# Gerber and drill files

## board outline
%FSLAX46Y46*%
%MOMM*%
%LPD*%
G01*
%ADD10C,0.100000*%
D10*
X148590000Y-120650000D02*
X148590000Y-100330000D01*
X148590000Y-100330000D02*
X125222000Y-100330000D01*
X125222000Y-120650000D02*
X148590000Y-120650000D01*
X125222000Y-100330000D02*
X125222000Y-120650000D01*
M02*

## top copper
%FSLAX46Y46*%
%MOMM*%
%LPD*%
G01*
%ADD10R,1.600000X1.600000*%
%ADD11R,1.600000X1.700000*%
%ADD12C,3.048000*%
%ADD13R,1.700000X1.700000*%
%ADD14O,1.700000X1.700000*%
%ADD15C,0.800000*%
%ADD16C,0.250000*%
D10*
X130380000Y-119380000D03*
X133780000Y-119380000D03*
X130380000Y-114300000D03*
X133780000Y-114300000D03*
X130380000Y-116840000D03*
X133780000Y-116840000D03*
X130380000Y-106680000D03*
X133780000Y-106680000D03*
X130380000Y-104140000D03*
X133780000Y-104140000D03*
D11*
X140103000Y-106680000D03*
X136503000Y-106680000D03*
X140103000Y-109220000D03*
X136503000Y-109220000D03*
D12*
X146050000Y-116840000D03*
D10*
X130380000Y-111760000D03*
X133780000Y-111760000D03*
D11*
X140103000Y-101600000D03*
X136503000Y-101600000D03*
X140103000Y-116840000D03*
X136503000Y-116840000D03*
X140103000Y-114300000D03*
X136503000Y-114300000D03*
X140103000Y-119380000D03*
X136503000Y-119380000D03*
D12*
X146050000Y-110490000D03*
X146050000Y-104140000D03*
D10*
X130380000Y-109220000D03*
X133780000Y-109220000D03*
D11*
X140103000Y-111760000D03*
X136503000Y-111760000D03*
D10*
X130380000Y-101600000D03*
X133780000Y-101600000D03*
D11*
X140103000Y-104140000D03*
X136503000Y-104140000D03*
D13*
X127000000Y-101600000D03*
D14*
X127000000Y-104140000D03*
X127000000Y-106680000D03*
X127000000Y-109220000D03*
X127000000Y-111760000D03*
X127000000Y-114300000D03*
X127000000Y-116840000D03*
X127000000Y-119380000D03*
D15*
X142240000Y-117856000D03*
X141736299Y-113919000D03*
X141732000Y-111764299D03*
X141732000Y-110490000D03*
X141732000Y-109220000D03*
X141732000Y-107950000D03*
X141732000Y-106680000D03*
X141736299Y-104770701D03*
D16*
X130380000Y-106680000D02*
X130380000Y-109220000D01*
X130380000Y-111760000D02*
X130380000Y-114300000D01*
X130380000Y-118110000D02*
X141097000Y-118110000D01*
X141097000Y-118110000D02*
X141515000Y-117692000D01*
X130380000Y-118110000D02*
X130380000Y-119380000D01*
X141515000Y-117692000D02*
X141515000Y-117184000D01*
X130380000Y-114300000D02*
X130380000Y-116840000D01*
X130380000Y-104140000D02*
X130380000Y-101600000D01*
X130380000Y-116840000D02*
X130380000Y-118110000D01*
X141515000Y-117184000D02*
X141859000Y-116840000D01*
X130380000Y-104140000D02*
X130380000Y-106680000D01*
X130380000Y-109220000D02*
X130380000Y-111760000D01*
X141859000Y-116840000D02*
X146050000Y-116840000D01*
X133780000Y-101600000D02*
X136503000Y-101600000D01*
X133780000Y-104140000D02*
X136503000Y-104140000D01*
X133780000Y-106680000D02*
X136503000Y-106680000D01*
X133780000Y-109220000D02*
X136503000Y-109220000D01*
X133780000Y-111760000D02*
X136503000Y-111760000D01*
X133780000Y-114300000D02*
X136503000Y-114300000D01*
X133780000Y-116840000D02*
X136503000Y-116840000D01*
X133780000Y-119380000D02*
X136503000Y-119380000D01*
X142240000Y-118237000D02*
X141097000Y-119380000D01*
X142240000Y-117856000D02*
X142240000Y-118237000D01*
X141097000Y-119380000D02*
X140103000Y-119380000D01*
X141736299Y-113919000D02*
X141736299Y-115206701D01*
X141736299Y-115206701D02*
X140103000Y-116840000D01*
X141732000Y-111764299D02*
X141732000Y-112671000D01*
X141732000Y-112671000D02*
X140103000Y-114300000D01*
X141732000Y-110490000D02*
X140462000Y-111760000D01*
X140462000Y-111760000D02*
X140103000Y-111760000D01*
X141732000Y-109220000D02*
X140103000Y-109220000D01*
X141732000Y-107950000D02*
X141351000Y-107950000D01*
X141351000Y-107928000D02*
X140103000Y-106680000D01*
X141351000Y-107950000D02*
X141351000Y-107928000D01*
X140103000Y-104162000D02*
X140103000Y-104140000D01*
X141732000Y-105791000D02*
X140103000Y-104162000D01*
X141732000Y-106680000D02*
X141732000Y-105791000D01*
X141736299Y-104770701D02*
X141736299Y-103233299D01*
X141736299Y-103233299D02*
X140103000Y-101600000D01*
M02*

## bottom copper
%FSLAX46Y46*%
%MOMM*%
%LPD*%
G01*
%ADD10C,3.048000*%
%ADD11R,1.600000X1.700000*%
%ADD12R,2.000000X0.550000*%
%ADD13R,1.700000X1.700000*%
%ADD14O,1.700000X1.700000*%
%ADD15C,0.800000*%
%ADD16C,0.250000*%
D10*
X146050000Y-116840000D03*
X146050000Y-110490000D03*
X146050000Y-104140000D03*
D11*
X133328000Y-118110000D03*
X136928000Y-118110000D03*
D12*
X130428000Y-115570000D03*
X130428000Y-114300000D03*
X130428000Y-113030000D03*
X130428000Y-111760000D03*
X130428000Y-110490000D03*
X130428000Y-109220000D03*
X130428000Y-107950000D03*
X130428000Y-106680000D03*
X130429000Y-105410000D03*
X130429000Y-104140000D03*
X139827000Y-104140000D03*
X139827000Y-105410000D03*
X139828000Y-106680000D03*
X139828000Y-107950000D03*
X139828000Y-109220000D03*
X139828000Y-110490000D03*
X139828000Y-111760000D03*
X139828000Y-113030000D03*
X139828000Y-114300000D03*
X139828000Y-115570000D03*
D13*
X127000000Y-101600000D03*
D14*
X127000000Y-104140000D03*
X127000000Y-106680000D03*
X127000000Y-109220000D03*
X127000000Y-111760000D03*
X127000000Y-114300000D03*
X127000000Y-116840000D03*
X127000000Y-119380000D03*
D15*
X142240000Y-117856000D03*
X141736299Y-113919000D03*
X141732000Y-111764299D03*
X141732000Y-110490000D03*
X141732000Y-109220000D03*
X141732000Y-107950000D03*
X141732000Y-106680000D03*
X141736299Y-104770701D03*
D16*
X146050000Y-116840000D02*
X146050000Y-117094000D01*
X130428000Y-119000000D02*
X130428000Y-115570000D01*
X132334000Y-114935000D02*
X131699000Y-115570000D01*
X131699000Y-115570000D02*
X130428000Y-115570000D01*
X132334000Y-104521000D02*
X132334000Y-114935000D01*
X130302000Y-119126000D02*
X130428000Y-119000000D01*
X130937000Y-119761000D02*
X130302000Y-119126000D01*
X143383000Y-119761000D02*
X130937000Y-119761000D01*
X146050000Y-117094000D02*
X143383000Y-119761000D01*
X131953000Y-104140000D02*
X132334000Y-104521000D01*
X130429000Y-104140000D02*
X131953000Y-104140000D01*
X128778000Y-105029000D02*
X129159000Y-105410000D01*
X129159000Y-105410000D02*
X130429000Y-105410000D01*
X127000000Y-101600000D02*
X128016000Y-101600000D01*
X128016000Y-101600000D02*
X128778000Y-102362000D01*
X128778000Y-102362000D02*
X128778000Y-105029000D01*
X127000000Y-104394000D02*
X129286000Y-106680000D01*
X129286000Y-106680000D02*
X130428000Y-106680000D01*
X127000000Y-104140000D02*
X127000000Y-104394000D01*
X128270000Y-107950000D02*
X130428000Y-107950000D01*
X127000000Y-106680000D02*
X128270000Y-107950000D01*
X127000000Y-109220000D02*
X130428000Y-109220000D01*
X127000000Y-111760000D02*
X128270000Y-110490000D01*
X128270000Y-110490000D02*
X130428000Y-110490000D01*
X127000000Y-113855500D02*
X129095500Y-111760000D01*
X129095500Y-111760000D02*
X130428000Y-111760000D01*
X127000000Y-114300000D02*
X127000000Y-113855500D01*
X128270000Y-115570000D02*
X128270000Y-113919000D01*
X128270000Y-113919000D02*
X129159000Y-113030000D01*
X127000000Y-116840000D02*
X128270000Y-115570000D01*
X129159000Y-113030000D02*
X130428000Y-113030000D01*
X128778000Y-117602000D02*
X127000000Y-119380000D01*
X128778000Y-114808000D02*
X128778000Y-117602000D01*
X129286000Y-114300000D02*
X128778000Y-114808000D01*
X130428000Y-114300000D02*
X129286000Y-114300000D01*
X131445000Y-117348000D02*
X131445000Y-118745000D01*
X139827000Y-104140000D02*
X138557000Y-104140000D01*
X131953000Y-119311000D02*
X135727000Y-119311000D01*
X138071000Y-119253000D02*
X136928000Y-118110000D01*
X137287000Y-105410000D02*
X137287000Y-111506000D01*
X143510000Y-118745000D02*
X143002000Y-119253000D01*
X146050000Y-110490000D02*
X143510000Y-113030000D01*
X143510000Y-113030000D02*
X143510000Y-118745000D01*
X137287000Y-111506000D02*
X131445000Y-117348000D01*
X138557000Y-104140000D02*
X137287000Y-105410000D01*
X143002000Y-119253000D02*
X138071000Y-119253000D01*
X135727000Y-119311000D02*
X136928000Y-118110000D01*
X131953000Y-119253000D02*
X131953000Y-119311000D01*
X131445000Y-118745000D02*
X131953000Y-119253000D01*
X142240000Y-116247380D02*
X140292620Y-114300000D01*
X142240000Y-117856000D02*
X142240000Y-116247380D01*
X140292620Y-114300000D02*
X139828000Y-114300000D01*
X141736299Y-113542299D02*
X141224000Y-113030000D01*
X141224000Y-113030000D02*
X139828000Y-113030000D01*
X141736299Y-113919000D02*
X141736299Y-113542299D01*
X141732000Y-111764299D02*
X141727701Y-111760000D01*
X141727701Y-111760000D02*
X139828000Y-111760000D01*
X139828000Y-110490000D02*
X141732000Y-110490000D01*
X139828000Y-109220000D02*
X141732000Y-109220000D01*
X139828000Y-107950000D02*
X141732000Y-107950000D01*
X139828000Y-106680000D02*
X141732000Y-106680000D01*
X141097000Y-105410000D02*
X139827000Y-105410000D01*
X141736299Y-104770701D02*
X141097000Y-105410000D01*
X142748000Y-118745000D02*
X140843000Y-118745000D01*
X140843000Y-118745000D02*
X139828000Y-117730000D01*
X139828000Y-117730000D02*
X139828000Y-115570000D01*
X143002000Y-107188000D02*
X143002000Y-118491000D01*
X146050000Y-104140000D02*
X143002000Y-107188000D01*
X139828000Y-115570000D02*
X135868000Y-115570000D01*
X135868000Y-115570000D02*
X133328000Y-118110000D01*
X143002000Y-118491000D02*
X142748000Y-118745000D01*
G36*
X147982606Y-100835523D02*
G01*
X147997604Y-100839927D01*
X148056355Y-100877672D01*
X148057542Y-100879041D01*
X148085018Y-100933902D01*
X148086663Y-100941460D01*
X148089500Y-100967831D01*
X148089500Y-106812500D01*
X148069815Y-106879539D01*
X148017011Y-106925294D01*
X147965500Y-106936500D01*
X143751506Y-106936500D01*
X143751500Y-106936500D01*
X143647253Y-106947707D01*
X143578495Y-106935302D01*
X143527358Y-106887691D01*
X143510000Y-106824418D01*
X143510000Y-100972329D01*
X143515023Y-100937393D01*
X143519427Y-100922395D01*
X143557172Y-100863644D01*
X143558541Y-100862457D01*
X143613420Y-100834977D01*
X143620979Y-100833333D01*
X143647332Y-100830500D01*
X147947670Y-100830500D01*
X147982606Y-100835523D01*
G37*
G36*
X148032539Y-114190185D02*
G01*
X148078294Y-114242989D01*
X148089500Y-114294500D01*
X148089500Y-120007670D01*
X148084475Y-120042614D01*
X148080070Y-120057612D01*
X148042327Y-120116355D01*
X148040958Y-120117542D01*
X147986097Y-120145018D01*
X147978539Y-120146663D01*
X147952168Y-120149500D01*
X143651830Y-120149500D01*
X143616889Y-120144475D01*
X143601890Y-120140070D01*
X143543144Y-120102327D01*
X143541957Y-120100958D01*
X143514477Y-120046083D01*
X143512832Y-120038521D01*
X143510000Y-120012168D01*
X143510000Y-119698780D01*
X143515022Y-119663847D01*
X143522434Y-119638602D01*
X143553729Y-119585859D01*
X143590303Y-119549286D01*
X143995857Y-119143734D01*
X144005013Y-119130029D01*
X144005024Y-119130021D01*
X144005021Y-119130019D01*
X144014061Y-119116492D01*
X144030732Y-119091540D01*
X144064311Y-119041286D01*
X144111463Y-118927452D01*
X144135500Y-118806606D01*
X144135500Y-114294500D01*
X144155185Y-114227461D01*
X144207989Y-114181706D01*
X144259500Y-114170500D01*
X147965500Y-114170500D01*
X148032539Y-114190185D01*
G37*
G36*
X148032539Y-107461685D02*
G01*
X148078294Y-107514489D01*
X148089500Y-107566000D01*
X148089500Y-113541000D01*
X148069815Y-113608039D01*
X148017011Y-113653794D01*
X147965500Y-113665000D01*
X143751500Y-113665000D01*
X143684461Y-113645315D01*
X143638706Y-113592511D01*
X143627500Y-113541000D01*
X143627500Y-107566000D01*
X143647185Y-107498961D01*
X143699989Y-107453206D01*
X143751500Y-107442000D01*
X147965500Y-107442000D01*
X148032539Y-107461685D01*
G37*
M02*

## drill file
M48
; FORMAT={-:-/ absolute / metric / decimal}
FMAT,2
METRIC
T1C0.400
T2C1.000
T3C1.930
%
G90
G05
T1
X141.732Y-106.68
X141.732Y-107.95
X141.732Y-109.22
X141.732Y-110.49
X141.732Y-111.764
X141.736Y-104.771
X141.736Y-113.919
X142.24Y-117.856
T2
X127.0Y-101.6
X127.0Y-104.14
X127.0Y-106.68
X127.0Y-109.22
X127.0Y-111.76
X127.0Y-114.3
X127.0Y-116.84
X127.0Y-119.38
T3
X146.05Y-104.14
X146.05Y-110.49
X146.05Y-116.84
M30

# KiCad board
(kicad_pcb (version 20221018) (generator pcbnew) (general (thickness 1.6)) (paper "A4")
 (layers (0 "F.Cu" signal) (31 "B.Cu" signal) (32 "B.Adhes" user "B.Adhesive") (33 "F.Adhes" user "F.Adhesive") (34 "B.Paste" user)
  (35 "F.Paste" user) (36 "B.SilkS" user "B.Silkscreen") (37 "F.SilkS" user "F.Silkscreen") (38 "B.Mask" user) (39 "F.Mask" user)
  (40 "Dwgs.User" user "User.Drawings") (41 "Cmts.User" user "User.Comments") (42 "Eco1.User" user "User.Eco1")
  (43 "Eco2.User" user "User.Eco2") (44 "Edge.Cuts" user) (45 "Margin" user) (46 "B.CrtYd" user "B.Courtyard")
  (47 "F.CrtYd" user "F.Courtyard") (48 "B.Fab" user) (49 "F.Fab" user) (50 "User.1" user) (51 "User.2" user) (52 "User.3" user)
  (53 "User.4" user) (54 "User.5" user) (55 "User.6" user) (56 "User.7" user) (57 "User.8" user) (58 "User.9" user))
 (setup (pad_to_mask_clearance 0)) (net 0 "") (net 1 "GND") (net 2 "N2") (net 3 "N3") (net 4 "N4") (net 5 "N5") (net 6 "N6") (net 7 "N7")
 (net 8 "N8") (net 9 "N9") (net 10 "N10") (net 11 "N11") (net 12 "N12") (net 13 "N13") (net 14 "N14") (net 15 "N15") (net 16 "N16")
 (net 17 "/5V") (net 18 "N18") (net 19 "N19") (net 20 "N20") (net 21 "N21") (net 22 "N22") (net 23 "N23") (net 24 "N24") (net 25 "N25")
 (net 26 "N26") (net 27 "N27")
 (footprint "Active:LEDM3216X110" (layer "F.Cu") (at 132.08 119.38)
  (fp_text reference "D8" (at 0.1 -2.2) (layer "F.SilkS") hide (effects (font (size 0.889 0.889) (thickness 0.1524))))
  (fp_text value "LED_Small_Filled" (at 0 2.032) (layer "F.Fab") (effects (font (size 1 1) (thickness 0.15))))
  (pad "1" smd rect (at -1.7 0 180) (size 1.6 1.6) (layers "F.Cu" "F.Paste" "F.Mask") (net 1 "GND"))
  (pad "2" smd rect (at 1.7 0 180) (size 1.6 1.6) (layers "F.Cu" "F.Paste" "F.Mask") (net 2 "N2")))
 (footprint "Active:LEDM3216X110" (layer "F.Cu") (at 132.08 114.3)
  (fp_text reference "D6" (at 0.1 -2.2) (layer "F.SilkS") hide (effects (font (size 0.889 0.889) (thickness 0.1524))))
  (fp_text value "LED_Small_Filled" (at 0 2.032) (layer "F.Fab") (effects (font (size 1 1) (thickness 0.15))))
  (pad "1" smd rect (at -1.7 0 180) (size 1.6 1.6) (layers "F.Cu" "F.Paste" "F.Mask") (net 1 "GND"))
  (pad "2" smd rect (at 1.7 0 180) (size 1.6 1.6) (layers "F.Cu" "F.Paste" "F.Mask") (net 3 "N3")))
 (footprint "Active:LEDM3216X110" (layer "F.Cu") (at 132.08 116.84)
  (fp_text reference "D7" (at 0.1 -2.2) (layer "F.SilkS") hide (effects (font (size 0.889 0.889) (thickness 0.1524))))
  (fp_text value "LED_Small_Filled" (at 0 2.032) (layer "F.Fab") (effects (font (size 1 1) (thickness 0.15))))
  (pad "1" smd rect (at -1.7 0 180) (size 1.6 1.6) (layers "F.Cu" "F.Paste" "F.Mask") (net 1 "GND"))
  (pad "2" smd rect (at 1.7 0 180) (size 1.6 1.6) (layers "F.Cu" "F.Paste" "F.Mask") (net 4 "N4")))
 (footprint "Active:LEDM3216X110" (layer "F.Cu") (at 132.08 106.68)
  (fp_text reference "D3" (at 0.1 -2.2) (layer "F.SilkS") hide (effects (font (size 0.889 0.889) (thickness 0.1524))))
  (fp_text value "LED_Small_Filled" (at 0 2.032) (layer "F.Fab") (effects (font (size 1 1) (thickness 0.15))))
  (pad "1" smd rect (at -1.7 0 180) (size 1.6 1.6) (layers "F.Cu" "F.Paste" "F.Mask") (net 1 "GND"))
  (pad "2" smd rect (at 1.7 0 180) (size 1.6 1.6) (layers "F.Cu" "F.Paste" "F.Mask") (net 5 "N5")))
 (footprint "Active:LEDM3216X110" (layer "F.Cu") (at 132.08 104.14)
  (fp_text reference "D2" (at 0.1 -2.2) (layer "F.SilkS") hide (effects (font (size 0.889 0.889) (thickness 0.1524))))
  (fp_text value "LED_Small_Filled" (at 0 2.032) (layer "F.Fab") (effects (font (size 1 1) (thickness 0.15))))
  (pad "1" smd rect (at -1.7 0 180) (size 1.6 1.6) (layers "F.Cu" "F.Paste" "F.Mask") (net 1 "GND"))
  (pad "2" smd rect (at 1.7 0 180) (size 1.6 1.6) (layers "F.Cu" "F.Paste" "F.Mask") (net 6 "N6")))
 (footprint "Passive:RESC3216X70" (layer "F.Cu") (at 138.303 106.68 180)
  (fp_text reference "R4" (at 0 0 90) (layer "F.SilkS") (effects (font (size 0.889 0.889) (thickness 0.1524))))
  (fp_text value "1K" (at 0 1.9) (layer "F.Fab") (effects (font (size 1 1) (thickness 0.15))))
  (pad "1" smd rect (at -1.8 0 180) (size 1.6 1.7) (layers "F.Cu" "F.Paste" "F.Mask") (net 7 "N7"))
  (pad "2" smd rect (at 1.8 0 180) (size 1.6 1.7) (layers "F.Cu" "F.Paste" "F.Mask") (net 5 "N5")))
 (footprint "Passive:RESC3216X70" (layer "F.Cu") (at 138.303 109.22 180)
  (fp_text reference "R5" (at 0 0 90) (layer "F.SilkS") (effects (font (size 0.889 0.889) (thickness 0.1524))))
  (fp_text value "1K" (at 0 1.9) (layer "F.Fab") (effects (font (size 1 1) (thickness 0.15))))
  (pad "1" smd rect (at -1.8 0 180) (size 1.6 1.7) (layers "F.Cu" "F.Paste" "F.Mask") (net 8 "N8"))
  (pad "2" smd rect (at 1.8 0 180) (size 1.6 1.7) (layers "F.Cu" "F.Paste" "F.Mask") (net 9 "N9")))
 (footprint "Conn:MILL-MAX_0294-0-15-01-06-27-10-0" (layer "F.Cu") (at 146.05 116.84)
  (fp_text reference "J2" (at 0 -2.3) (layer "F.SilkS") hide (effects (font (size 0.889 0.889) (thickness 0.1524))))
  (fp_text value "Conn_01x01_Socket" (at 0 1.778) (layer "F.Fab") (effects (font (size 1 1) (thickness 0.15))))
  (pad "1" thru_hole circle (at 0 0) (size 3.048 3.048) (drill 1.9304) (layers "*.Cu" "*.Mask") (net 1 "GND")))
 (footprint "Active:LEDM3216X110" (layer "F.Cu") (at 132.08 111.76)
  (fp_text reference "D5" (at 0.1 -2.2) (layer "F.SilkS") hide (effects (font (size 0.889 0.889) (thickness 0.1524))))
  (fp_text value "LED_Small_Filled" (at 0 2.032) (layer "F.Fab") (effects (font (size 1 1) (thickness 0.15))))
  (pad "1" smd rect (at -1.7 0 180) (size 1.6 1.6) (layers "F.Cu" "F.Paste" "F.Mask") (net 1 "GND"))
  (pad "2" smd rect (at 1.7 0 180) (size 1.6 1.6) (layers "F.Cu" "F.Paste" "F.Mask") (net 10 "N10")))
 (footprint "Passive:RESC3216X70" (layer "F.Cu") (at 138.303 101.6 180)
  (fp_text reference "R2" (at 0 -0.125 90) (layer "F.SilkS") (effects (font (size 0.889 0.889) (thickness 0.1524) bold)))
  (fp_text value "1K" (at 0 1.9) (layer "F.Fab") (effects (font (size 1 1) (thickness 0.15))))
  (pad "1" smd rect (at -1.8 0 180) (size 1.6 1.7) (layers "F.Cu" "F.Paste" "F.Mask") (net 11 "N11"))
  (pad "2" smd rect (at 1.8 0 180) (size 1.6 1.7) (layers "F.Cu" "F.Paste" "F.Mask") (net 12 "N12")))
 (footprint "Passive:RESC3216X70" (layer "F.Cu") (at 138.303 116.84 180)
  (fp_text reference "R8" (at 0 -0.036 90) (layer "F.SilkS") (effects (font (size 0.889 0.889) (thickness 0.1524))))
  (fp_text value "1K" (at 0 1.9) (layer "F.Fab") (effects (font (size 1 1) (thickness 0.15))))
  (pad "1" smd rect (at -1.8 0 180) (size 1.6 1.7) (layers "F.Cu" "F.Paste" "F.Mask") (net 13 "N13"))
  (pad "2" smd rect (at 1.8 0 180) (size 1.6 1.7) (layers "F.Cu" "F.Paste" "F.Mask") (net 4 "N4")))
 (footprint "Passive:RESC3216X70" (layer "F.Cu") (at 138.303 114.3 180)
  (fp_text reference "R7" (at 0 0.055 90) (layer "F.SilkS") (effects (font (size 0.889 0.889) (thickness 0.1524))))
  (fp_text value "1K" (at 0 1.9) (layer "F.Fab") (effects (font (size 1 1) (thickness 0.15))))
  (pad "1" smd rect (at -1.8 0 180) (size 1.6 1.7) (layers "F.Cu" "F.Paste" "F.Mask") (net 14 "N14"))
  (pad "2" smd rect (at 1.8 0 180) (size 1.6 1.7) (layers "F.Cu" "F.Paste" "F.Mask") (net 3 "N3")))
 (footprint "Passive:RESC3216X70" (layer "F.Cu") (at 138.303 119.38 180)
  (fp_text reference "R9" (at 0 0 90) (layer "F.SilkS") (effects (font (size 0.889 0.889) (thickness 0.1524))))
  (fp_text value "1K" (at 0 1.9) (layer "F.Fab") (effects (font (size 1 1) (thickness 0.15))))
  (pad "1" smd rect (at -1.8 0 180) (size 1.6 1.7) (layers "F.Cu" "F.Paste" "F.Mask") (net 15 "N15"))
  (pad "2" smd rect (at 1.8 0 180) (size 1.6 1.7) (layers "F.Cu" "F.Paste" "F.Mask") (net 2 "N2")))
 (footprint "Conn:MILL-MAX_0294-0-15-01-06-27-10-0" (layer "F.Cu") (at 146.05 110.49)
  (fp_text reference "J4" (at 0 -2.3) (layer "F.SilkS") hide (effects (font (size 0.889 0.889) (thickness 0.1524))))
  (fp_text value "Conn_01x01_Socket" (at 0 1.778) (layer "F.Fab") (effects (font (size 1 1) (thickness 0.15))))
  (pad "1" thru_hole circle (at 0 0) (size 3.048 3.048) (drill 1.9304) (layers "*.Cu" "*.Mask") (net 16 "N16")))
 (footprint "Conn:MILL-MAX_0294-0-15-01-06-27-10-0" (layer "F.Cu") (at 146.05 104.14)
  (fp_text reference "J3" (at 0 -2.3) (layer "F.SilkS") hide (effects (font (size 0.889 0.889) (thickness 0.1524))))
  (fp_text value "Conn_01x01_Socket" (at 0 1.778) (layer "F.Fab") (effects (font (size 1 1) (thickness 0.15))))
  (pad "1" thru_hole circle (at 0 0) (size 3.048 3.048) (drill 1.9304) (layers "*.Cu" "*.Mask") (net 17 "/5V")))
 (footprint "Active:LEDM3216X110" (layer "F.Cu") (at 132.08 109.22)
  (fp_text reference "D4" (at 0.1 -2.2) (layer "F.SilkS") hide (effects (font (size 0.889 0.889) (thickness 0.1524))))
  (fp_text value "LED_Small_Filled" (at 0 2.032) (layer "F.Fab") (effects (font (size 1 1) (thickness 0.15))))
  (pad "1" smd rect (at -1.7 0 180) (size 1.6 1.6) (layers "F.Cu" "F.Paste" "F.Mask") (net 1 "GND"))
  (pad "2" smd rect (at 1.7 0 180) (size 1.6 1.6) (layers "F.Cu" "F.Paste" "F.Mask") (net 9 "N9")))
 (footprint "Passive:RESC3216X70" (layer "F.Cu") (at 138.303 111.76 180)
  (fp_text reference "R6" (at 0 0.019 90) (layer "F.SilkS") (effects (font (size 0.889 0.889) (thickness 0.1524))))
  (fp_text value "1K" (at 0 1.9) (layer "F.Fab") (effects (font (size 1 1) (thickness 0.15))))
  (pad "1" smd rect (at -1.8 0 180) (size 1.6 1.7) (layers "F.Cu" "F.Paste" "F.Mask") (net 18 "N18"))
  (pad "2" smd rect (at 1.8 0 180) (size 1.6 1.7) (layers "F.Cu" "F.Paste" "F.Mask") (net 10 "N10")))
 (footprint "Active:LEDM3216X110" (layer "F.Cu") (at 132.08 101.6)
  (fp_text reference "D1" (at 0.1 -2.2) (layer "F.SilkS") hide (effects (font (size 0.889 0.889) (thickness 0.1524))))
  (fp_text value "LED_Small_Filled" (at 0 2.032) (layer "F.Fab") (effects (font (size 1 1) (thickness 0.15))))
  (pad "1" smd rect (at -1.7 0 180) (size 1.6 1.6) (layers "F.Cu" "F.Paste" "F.Mask") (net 1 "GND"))
  (pad "2" smd rect (at 1.7 0 180) (size 1.6 1.6) (layers "F.Cu" "F.Paste" "F.Mask") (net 12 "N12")))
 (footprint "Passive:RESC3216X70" (layer "F.Cu") (at 138.303 104.14 180)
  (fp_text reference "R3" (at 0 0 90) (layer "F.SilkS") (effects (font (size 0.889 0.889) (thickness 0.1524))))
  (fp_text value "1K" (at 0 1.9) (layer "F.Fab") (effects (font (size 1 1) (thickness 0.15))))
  (pad "1" smd rect (at -1.8 0 180) (size 1.6 1.7) (layers "F.Cu" "F.Paste" "F.Mask") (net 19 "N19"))
  (pad "2" smd rect (at 1.8 0 180) (size 1.6 1.7) (layers "F.Cu" "F.Paste" "F.Mask") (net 6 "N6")))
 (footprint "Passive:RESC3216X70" (layer "B.Cu") (at 135.128 118.11)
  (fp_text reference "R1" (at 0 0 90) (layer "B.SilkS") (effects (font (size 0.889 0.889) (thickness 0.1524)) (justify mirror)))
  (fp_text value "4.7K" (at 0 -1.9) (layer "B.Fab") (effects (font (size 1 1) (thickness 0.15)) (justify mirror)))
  (pad "1" smd rect (at -1.8 0) (size 1.6 1.7) (layers "B.Cu" "B.Paste" "B.Mask") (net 17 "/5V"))
  (pad "2" smd rect (at 1.8 0) (size 1.6 1.7) (layers "B.Cu" "B.Paste" "B.Mask") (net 16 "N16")))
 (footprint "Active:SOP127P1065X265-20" (layer "B.Cu") (at 135.128 109.855)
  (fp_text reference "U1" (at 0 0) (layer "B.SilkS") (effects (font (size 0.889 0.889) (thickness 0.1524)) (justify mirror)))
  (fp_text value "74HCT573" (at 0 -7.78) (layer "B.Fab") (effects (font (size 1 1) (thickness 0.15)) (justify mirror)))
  (pad "1" smd rect (at -4.7 5.715) (size 2 0.55) (layers "B.Cu" "B.Paste" "B.Mask") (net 1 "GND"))
  (pad "2" smd rect (at -4.7 4.445) (size 2 0.55) (layers "B.Cu" "B.Paste" "B.Mask") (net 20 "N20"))
  (pad "3" smd rect (at -4.7 3.175) (size 2 0.55) (layers "B.Cu" "B.Paste" "B.Mask") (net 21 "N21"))
  (pad "4" smd rect (at -4.7 1.905) (size 2 0.55) (layers "B.Cu" "B.Paste" "B.Mask") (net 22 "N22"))
  (pad "5" smd rect (at -4.7 0.635) (size 2 0.55) (layers "B.Cu" "B.Paste" "B.Mask") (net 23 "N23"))
  (pad "6" smd rect (at -4.7 -0.635) (size 2 0.55) (layers "B.Cu" "B.Paste" "B.Mask") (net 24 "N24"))
  (pad "7" smd rect (at -4.7 -1.905) (size 2 0.55) (layers "B.Cu" "B.Paste" "B.Mask") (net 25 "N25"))
  (pad "8" smd rect (at -4.7 -3.175) (size 2 0.55) (layers "B.Cu" "B.Paste" "B.Mask") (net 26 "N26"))
  (pad "9" smd rect (at -4.699 -4.445) (size 2 0.55) (layers "B.Cu" "B.Paste" "B.Mask") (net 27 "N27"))
  (pad "10" smd rect (at -4.699 -5.715) (size 2 0.55) (layers "B.Cu" "B.Paste" "B.Mask") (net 1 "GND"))
  (pad "11" smd rect (at 4.699 -5.715) (size 2 0.55) (layers "B.Cu" "B.Paste" "B.Mask") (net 16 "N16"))
  (pad "12" smd rect (at 4.699 -4.445) (size 2 0.55) (layers "B.Cu" "B.Paste" "B.Mask") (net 11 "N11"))
  (pad "13" smd rect (at 4.7 -3.175) (size 2 0.55) (layers "B.Cu" "B.Paste" "B.Mask") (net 19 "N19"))
  (pad "14" smd rect (at 4.7 -1.905) (size 2 0.55) (layers "B.Cu" "B.Paste" "B.Mask") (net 7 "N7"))
  (pad "15" smd rect (at 4.7 -0.635) (size 2 0.55) (layers "B.Cu" "B.Paste" "B.Mask") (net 8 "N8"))
  (pad "16" smd rect (at 4.7 0.635) (size 2 0.55) (layers "B.Cu" "B.Paste" "B.Mask") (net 18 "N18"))
  (pad "17" smd rect (at 4.7 1.905) (size 2 0.55) (layers "B.Cu" "B.Paste" "B.Mask") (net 14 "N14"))
  (pad "18" smd rect (at 4.7 3.175) (size 2 0.55) (layers "B.Cu" "B.Paste" "B.Mask") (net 13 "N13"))
  (pad "19" smd rect (at 4.7 4.445) (size 2 0.55) (layers "B.Cu" "B.Paste" "B.Mask") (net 15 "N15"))
  (pad "20" smd rect (at 4.7 5.715) (size 2 0.55) (layers "B.Cu" "B.Paste" "B.Mask") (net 17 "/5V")))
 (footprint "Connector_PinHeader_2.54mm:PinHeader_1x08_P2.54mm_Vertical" (layer "B.Cu") (at 127 101.6 180)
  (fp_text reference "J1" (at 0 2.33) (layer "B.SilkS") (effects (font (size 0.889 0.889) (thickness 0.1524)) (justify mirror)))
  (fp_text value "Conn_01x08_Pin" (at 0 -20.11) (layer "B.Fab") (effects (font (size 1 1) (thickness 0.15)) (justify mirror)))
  (pad "1" thru_hole rect (at 0 0 180) (size 1.7 1.7) (drill 1) (layers "*.Cu" "*.Mask") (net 27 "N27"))
  (pad "2" thru_hole oval (at 0 -2.54 180) (size 1.7 1.7) (drill 1) (layers "*.Cu" "*.Mask") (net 26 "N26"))
  (pad "3" thru_hole oval (at 0 -5.08 180) (size 1.7 1.7) (drill 1) (layers "*.Cu" "*.Mask") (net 25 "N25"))
  (pad "4" thru_hole oval (at 0 -7.62 180) (size 1.7 1.7) (drill 1) (layers "*.Cu" "*.Mask") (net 24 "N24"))
  (pad "5" thru_hole oval (at 0 -10.16 180) (size 1.7 1.7) (drill 1) (layers "*.Cu" "*.Mask") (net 23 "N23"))
  (pad "6" thru_hole oval (at 0 -12.7 180) (size 1.7 1.7) (drill 1) (layers "*.Cu" "*.Mask") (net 22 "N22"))
  (pad "7" thru_hole oval (at 0 -15.24 180) (size 1.7 1.7) (drill 1) (layers "*.Cu" "*.Mask") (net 21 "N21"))
  (pad "8" thru_hole oval (at 0 -17.78 180) (size 1.7 1.7) (drill 1) (layers "*.Cu" "*.Mask") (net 20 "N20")))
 (gr_line (start 148.59 120.65) (end 148.59 100.33) (stroke (width 0.1) (type default)) (layer "Edge.Cuts"))
 (gr_line (start 148.59 100.33) (end 125.222 100.33) (stroke (width 0.1) (type default)) (layer "Edge.Cuts"))
 (gr_line (start 125.222 120.65) (end 148.59 120.65) (stroke (width 0.1) (type default)) (layer "Edge.Cuts"))
 (gr_line (start 125.222 100.33) (end 125.222 120.65) (stroke (width 0.1) (type default)) (layer "Edge.Cuts"))
 (segment (start 130.38 106.68) (end 130.38 109.22) (width 0.25) (layer "F.Cu") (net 1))
 (segment (start 130.38 111.76) (end 130.38 114.3) (width 0.25) (layer "F.Cu") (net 1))
 (segment (start 130.38 118.11) (end 141.097 118.11) (width 0.25) (layer "F.Cu") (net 1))
 (segment (start 141.097 118.11) (end 141.515 117.692) (width 0.25) (layer "F.Cu") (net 1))
 (segment (start 130.38 118.11) (end 130.38 119.38) (width 0.25) (layer "F.Cu") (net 1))
 (segment (start 141.515 117.692) (end 141.515 117.184) (width 0.25) (layer "F.Cu") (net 1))
 (segment (start 130.38 114.3) (end 130.38 116.84) (width 0.25) (layer "F.Cu") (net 1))
 (segment (start 130.38 104.14) (end 130.38 101.6) (width 0.25) (layer "F.Cu") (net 1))
 (segment (start 130.38 116.84) (end 130.38 118.11) (width 0.25) (layer "F.Cu") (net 1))
 (segment (start 141.515 117.184) (end 141.859 116.84) (width 0.25) (layer "F.Cu") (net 1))
 (segment (start 130.38 104.14) (end 130.38 106.68) (width 0.25) (layer "F.Cu") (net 1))
 (segment (start 130.38 109.22) (end 130.38 111.76) (width 0.25) (layer "F.Cu") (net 1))
 (segment (start 141.859 116.84) (end 146.05 116.84) (width 0.25) (layer "F.Cu") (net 1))
 (segment (start 146.05 116.84) (end 146.05 117.094) (width 0.25) (layer "B.Cu") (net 1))
 (segment (start 130.428 119) (end 130.428 115.57) (width 0.25) (layer "B.Cu") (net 1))
 (segment (start 132.334 114.935) (end 131.699 115.57) (width 0.25) (layer "B.Cu") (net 1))
 (segment (start 131.699 115.57) (end 130.428 115.57) (width 0.25) (layer "B.Cu") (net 1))
 (segment (start 132.334 104.521) (end 132.334 114.935) (width 0.25) (layer "B.Cu") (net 1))
 (segment (start 130.302 119.126) (end 130.428 119) (width 0.25) (layer "B.Cu") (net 1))
 (segment (start 130.937 119.761) (end 130.302 119.126) (width 0.25) (layer "B.Cu") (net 1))
 (segment (start 143.383 119.761) (end 130.937 119.761) (width 0.25) (layer "B.Cu") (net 1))
 (segment (start 146.05 117.094) (end 143.383 119.761) (width 0.25) (layer "B.Cu") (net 1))
 (segment (start 131.953 104.14) (end 132.334 104.521) (width 0.25) (layer "B.Cu") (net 1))
 (segment (start 130.429 104.14) (end 131.953 104.14) (width 0.25) (layer "B.Cu") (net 1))
 (segment (start 133.78 101.6) (end 136.503 101.6) (width 0.25) (layer "F.Cu") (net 12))
 (segment (start 133.78 104.14) (end 136.503 104.14) (width 0.25) (layer "F.Cu") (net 6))
 (segment (start 133.78 106.68) (end 136.503 106.68) (width 0.25) (layer "F.Cu") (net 5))
 (segment (start 133.78 109.22) (end 136.503 109.22) (width 0.25) (layer "F.Cu") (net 9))
 (segment (start 133.78 111.76) (end 136.503 111.76) (width 0.25) (layer "F.Cu") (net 10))
 (segment (start 133.78 114.3) (end 136.503 114.3) (width 0.25) (layer "F.Cu") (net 3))
 (segment (start 133.78 116.84) (end 136.503 116.84) (width 0.25) (layer "F.Cu") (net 4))
 (segment (start 133.78 119.38) (end 136.503 119.38) (width 0.25) (layer "F.Cu") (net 2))
 (segment (start 128.778 105.029) (end 129.159 105.41) (width 0.25) (layer "B.Cu") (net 27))
 (segment (start 129.159 105.41) (end 130.429 105.41) (width 0.25) (layer "B.Cu") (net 27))
 (segment (start 127 101.6) (end 128.016 101.6) (width 0.25) (layer "B.Cu") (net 27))
 (segment (start 128.016 101.6) (end 128.778 102.362) (width 0.25) (layer "B.Cu") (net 27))
 (segment (start 128.778 102.362) (end 128.778 105.029) (width 0.25) (layer "B.Cu") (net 27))
 (segment (start 127 104.394) (end 129.286 106.68) (width 0.25) (layer "B.Cu") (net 26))
 (segment (start 129.286 106.68) (end 130.428 106.68) (width 0.25) (layer "B.Cu") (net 26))
 (segment (start 127 104.14) (end 127 104.394) (width 0.25) (layer "B.Cu") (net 26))
 (segment (start 128.27 107.95) (end 130.428 107.95) (width 0.25) (layer "B.Cu") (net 25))
 (segment (start 127 106.68) (end 128.27 107.95) (width 0.25) (layer "B.Cu") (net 25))
 (segment (start 127 109.22) (end 130.428 109.22) (width 0.25) (layer "B.Cu") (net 24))
 (segment (start 127 111.76) (end 128.27 110.49) (width 0.25) (layer "B.Cu") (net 23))
 (segment (start 128.27 110.49) (end 130.428 110.49) (width 0.25) (layer "B.Cu") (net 23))
 (segment (start 127 113.8555) (end 129.0955 111.76) (width 0.25) (layer "B.Cu") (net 22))
 (segment (start 129.0955 111.76) (end 130.428 111.76) (width 0.25) (layer "B.Cu") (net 22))
 (segment (start 127 114.3) (end 127 113.8555) (width 0.25) (layer "B.Cu") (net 22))
 (segment (start 128.27 115.57) (end 128.27 113.919) (width 0.25) (layer "B.Cu") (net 21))
 (segment (start 128.27 113.919) (end 129.159 113.03) (width 0.25) (layer "B.Cu") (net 21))
 (segment (start 127 116.84) (end 128.27 115.57) (width 0.25) (layer "B.Cu") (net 21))
 (segment (start 129.159 113.03) (end 130.428 113.03) (width 0.25) (layer "B.Cu") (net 21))
 (segment (start 128.778 117.602) (end 127 119.38) (width 0.25) (layer "B.Cu") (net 20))
 (segment (start 128.778 114.808) (end 128.778 117.602) (width 0.25) (layer "B.Cu") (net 20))
 (segment (start 129.286 114.3) (end 128.778 114.808) (width 0.25) (layer "B.Cu") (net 20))
 (segment (start 130.428 114.3) (end 129.286 114.3) (width 0.25) (layer "B.Cu") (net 20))
 (segment (start 131.445 117.348) (end 131.445 118.745) (width 0.25) (layer "B.Cu") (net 16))
 (segment (start 139.827 104.14) (end 138.557 104.14) (width 0.25) (layer "B.Cu") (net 16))
 (segment (start 131.953 119.311) (end 135.727 119.311) (width 0.25) (layer "B.Cu") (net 16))
 (segment (start 138.071 119.253) (end 136.928 118.11) (width 0.25) (layer "B.Cu") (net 16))
 (segment (start 137.287 105.41) (end 137.287 111.506) (width 0.25) (layer "B.Cu") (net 16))
 (segment (start 143.51 118.745) (end 143.002 119.253) (width 0.25) (layer "B.Cu") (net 16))
 (segment (start 146.05 110.49) (end 143.51 113.03) (width 0.25) (layer "B.Cu") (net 16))
 (segment (start 143.51 113.03) (end 143.51 118.745) (width 0.25) (layer "B.Cu") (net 16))
 (segment (start 137.287 111.506) (end 131.445 117.348) (width 0.25) (layer "B.Cu") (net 16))
 (segment (start 138.557 104.14) (end 137.287 105.41) (width 0.25) (layer "B.Cu") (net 16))
 (segment (start 143.002 119.253) (end 138.071 119.253) (width 0.25) (layer "B.Cu") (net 16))
 (segment (start 135.727 119.311) (end 136.928 118.11) (width 0.25) (layer "B.Cu") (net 16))
 (segment (start 131.953 119.253) (end 131.953 119.311) (width 0.25) (layer "B.Cu") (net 16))
 (segment (start 131.445 118.745) (end 131.953 119.253) (width 0.25) (layer "B.Cu") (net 16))
 (segment (start 142.24 118.237) (end 141.097 119.38) (width 0.25) (layer "F.Cu") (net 15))
 (segment (start 142.24 117.856) (end 142.24 118.237) (width 0.25) (layer "F.Cu") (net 15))
 (segment (start 141.097 119.38) (end 140.103 119.38) (width 0.25) (layer "F.Cu") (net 15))
 (via (at 142.24 117.856) (size 0.8) (drill 0.4) (layers "F.Cu" "B.Cu") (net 15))
 (segment (start 142.24 116.24738) (end 140.29262 114.3) (width 0.25) (layer "B.Cu") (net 15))
 (segment (start 142.24 117.856) (end 142.24 116.24738) (width 0.25) (layer "B.Cu") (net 15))
 (segment (start 140.29262 114.3) (end 139.828 114.3) (width 0.25) (layer "B.Cu") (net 15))
 (segment (start 141.736299 113.919) (end 141.736299 115.206701) (width 0.25) (layer "F.Cu") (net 13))
 (segment (start 141.736299 115.206701) (end 140.103 116.84) (width 0.25) (layer "F.Cu") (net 13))
 (via (at 141.736299 113.919) (size 0.8) (drill 0.4) (layers "F.Cu" "B.Cu") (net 13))
 (segment (start 141.736299 113.542299) (end 141.224 113.03) (width 0.25) (layer "B.Cu") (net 13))
 (segment (start 141.224 113.03) (end 139.828 113.03) (width 0.25) (layer "B.Cu") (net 13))
 (segment (start 141.736299 113.919) (end 141.736299 113.542299) (width 0.25) (layer "B.Cu") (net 13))
 (segment (start 141.732 111.764299) (end 141.732 112.671) (width 0.25) (layer "F.Cu") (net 14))
 (segment (start 141.732 112.671) (end 140.103 114.3) (width 0.25) (layer "F.Cu") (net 14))
 (via (at 141.732 111.764299) (size 0.8) (drill 0.4) (layers "F.Cu" "B.Cu") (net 14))
 (segment (start 141.732 111.764299) (end 141.727701 111.76) (width 0.25) (layer "B.Cu") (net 14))
 (segment (start 141.727701 111.76) (end 139.828 111.76) (width 0.25) (layer "B.Cu") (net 14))
 (segment (start 141.732 110.49) (end 140.462 111.76) (width 0.25) (layer "F.Cu") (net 18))
 (segment (start 140.462 111.76) (end 140.103 111.76) (width 0.25) (layer "F.Cu") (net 18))
 (via (at 141.732 110.49) (size 0.8) (drill 0.4) (layers "F.Cu" "B.Cu") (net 18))
 (segment (start 139.828 110.49) (end 141.732 110.49) (width 0.25) (layer "B.Cu") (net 18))
 (segment (start 141.732 109.22) (end 140.103 109.22) (width 0.25) (layer "F.Cu") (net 8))
 (via (at 141.732 109.22) (size 0.8) (drill 0.4) (layers "F.Cu" "B.Cu") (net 8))
 (segment (start 139.828 109.22) (end 141.732 109.22) (width 0.25) (layer "B.Cu") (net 8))
 (segment (start 141.732 107.95) (end 141.351 107.95) (width 0.25) (layer "F.Cu") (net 7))
 (segment (start 141.351 107.928) (end 140.103 106.68) (width 0.25) (layer "F.Cu") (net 7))
 (segment (start 141.351 107.95) (end 141.351 107.928) (width 0.25) (layer "F.Cu") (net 7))
 (via (at 141.732 107.95) (size 0.8) (drill 0.4) (layers "F.Cu" "B.Cu") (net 7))
 (segment (start 139.828 107.95) (end 141.732 107.95) (width 0.25) (layer "B.Cu") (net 7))
 (segment (start 140.103 104.162) (end 140.103 104.14) (width 0.25) (layer "F.Cu") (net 19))
 (segment (start 141.732 105.791) (end 140.103 104.162) (width 0.25) (layer "F.Cu") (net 19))
 (segment (start 141.732 106.68) (end 141.732 105.791) (width 0.25) (layer "F.Cu") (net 19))
 (via (at 141.732 106.68) (size 0.8) (drill 0.4) (layers "F.Cu" "B.Cu") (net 19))
 (segment (start 139.828 106.68) (end 141.732 106.68) (width 0.25) (layer "B.Cu") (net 19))
 (segment (start 141.736299 104.770701) (end 141.736299 103.233299) (width 0.25) (layer "F.Cu") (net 11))
 (segment (start 141.736299 103.233299) (end 140.103 101.6) (width 0.25) (layer "F.Cu") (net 11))
 (via (at 141.736299 104.770701) (size 0.8) (drill 0.4) (layers "F.Cu" "B.Cu") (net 11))
 (segment (start 141.097 105.41) (end 139.827 105.41) (width 0.25) (layer "B.Cu") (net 11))
 (segment (start 141.736299 104.770701) (end 141.097 105.41) (width 0.25) (layer "B.Cu") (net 11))
 (segment (start 142.748 118.745) (end 140.843 118.745) (width 0.25) (layer "B.Cu") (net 17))
 (segment (start 140.843 118.745) (end 139.828 117.73) (width 0.25) (layer "B.Cu") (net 17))
 (segment (start 139.828 117.73) (end 139.828 115.57) (width 0.25) (layer "B.Cu") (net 17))
 (segment (start 143.002 107.188) (end 143.002 118.491) (width 0.25) (layer "B.Cu") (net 17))
 (segment (start 146.05 104.14) (end 143.002 107.188) (width 0.25) (layer "B.Cu") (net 17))
 (segment (start 139.828 115.57) (end 135.868 115.57) (width 0.25) (layer "B.Cu") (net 17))
 (segment (start 135.868 115.57) (end 133.328 118.11) (width 0.25) (layer "B.Cu") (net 17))
 (segment (start 143.002 118.491) (end 142.748 118.745) (width 0.25) (layer "B.Cu") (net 17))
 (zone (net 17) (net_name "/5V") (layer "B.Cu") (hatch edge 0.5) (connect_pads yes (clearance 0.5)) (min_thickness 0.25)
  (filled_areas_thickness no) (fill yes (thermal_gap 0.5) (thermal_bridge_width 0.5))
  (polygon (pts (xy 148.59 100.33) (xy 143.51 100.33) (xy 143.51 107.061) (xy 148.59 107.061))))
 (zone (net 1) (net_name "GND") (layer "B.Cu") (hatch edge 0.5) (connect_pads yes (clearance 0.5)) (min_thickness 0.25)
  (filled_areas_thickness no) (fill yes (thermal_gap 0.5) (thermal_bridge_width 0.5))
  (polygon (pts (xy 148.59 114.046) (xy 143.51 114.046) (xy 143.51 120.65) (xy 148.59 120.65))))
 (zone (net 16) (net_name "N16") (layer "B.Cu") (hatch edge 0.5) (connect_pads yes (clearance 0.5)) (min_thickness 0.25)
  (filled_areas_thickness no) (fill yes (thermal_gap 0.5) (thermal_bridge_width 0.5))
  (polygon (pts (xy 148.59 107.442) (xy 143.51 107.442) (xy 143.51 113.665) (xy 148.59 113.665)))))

